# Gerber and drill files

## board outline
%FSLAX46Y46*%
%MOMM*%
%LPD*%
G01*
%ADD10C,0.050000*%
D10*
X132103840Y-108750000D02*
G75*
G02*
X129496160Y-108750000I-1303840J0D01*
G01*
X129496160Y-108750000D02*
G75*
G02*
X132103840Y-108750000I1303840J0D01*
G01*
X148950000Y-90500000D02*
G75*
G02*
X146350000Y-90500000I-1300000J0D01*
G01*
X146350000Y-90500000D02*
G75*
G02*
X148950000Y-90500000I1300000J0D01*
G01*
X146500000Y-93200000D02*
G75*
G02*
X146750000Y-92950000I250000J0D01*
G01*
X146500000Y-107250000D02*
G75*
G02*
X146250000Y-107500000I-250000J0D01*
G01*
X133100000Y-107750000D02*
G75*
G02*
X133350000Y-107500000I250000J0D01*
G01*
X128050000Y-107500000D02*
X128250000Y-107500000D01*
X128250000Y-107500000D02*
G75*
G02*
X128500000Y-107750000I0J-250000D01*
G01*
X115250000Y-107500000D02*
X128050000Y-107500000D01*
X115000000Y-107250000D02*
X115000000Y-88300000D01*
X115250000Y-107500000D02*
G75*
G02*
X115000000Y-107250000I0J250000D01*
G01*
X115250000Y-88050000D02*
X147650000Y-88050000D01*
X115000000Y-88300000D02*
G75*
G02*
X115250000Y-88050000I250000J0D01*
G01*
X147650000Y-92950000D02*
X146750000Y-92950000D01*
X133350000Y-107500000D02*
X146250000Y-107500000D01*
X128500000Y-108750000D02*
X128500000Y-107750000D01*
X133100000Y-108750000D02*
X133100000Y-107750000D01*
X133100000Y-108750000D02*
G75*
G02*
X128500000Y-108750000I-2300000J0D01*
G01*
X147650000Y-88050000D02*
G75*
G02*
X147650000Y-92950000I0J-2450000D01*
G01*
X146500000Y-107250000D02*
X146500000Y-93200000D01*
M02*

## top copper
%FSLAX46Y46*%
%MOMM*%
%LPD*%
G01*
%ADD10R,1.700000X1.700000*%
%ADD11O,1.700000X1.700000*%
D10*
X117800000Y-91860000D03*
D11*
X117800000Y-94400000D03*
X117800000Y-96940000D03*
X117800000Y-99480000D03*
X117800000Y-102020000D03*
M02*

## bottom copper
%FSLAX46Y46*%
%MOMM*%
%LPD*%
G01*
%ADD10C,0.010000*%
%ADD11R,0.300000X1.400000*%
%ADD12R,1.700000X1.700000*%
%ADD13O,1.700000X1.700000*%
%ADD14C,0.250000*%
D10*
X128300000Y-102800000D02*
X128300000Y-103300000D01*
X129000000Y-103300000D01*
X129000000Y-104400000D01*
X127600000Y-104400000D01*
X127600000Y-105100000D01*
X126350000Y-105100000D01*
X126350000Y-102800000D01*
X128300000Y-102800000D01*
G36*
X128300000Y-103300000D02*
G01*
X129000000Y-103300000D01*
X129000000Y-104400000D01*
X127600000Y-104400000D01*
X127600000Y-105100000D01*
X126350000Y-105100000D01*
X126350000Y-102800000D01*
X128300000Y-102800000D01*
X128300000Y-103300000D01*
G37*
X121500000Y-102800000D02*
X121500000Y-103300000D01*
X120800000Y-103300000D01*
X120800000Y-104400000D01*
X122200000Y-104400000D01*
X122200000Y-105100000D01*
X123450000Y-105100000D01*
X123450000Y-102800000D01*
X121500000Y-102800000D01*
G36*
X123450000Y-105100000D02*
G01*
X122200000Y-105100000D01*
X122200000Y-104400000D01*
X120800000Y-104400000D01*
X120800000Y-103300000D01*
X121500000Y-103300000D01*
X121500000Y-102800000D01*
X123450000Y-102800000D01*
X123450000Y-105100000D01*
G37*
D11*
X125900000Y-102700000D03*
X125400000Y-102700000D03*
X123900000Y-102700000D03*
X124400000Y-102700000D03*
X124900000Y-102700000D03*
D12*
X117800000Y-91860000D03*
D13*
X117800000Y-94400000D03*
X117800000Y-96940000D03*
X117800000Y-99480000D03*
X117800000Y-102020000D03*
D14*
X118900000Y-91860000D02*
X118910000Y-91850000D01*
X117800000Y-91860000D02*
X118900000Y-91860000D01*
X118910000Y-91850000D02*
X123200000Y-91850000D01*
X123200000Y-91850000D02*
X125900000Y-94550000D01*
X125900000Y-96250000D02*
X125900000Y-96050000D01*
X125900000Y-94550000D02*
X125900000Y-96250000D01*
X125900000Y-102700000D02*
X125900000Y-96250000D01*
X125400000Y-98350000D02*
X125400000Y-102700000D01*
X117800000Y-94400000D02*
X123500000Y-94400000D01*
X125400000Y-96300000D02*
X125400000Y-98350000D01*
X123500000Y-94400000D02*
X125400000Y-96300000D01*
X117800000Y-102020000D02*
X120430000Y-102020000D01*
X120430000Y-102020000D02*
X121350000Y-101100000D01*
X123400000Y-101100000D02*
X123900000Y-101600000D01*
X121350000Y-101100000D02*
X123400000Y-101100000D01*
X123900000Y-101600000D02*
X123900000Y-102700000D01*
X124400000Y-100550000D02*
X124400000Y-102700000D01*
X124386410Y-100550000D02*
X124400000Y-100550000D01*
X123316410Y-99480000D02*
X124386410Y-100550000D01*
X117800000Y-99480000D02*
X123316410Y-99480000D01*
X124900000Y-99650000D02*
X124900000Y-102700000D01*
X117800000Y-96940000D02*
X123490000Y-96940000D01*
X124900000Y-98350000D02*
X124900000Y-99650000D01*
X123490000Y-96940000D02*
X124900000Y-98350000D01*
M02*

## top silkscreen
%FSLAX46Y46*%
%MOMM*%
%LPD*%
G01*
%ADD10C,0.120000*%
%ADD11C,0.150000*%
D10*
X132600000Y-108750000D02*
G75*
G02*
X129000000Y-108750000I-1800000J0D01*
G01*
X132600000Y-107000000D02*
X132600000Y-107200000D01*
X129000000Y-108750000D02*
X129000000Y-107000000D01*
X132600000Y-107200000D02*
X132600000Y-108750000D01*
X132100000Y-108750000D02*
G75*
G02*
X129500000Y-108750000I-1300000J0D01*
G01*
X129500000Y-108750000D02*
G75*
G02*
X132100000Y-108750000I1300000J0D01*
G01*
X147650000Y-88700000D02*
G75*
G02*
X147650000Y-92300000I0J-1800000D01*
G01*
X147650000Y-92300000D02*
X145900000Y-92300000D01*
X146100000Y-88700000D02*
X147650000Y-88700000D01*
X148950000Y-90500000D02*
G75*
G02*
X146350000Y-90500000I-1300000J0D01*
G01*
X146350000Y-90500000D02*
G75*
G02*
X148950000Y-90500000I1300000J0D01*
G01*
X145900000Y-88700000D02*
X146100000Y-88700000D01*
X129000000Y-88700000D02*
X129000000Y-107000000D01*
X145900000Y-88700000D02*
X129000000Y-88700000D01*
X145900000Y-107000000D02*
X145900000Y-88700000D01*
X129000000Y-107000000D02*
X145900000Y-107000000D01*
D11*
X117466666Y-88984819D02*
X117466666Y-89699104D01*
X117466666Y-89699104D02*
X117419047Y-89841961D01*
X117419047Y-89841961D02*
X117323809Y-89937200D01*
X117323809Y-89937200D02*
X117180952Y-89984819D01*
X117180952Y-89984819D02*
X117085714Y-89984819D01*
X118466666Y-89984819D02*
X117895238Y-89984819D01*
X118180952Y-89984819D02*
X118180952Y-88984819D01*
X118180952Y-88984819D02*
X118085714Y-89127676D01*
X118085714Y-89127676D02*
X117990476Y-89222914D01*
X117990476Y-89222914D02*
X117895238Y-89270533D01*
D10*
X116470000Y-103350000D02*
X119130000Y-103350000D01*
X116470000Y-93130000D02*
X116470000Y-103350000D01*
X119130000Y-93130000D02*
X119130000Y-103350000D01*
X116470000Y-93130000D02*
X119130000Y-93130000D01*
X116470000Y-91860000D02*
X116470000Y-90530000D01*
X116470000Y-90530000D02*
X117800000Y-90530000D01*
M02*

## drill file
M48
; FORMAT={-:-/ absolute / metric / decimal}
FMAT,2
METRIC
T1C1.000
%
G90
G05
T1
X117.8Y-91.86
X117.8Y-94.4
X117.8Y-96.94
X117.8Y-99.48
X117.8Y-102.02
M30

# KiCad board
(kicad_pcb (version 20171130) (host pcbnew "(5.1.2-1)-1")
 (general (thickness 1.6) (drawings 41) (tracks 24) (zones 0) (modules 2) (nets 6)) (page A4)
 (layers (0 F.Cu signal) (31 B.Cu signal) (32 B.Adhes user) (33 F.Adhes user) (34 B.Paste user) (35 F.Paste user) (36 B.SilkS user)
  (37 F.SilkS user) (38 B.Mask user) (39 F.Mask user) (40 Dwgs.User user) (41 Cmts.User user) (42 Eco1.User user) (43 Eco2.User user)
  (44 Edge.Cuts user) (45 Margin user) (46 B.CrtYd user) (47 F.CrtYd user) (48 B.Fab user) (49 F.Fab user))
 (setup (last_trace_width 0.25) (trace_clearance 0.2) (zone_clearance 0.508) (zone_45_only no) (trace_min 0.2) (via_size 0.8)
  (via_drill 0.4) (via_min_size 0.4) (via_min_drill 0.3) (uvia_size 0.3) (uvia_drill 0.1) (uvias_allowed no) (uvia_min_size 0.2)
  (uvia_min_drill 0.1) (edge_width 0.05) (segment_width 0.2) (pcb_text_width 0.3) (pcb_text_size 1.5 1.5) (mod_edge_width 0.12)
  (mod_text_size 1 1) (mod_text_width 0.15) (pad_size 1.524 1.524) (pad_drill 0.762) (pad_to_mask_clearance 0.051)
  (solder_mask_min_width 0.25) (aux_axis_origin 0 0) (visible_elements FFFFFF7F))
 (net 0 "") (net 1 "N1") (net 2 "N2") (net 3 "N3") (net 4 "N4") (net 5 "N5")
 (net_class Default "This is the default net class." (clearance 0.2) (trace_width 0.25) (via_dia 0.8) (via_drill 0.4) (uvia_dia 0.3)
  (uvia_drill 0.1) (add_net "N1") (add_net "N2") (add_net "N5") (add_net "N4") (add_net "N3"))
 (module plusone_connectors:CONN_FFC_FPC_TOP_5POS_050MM (layer B.Cu) (at 124.9 105.2 180)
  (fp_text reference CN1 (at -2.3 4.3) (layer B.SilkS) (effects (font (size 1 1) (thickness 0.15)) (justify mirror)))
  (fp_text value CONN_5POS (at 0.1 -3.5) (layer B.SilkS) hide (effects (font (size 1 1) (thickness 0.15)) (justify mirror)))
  (fp_poly
   (pts (xy -3.4 2.4) (xy -3.4 1.9) (xy -4.1 1.9) (xy -4.1 0.8) (xy -2.7 0.8) (xy -2.7 0.1) (xy -1.45 0.1) (xy -1.45 2.4)) (layer B.Cu)
   (width 0.01))
  (fp_poly
   (pts (xy 3.4 2.4) (xy 3.4 1.9) (xy 4.1 1.9) (xy 4.1 0.8) (xy 2.7 0.8) (xy 2.7 0.1) (xy 1.45 0.1) (xy 1.45 2.4)) (layer B.Cu) (width 0.01))
  (pad 1 smd rect (at -1 2.5 180) (size 0.3 1.4) (layers B.Cu B.Paste B.Mask) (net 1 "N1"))
  (pad 2 smd rect (at -0.5 2.5 180) (size 0.3 1.4) (layers B.Cu B.Paste B.Mask) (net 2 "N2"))
  (pad 5 smd rect (at 1 2.5 180) (size 0.3 1.4) (layers B.Cu B.Paste B.Mask) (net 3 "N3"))
  (pad 4 smd rect (at 0.5 2.5 180) (size 0.3 1.4) (layers B.Cu B.Paste B.Mask) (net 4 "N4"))
  (pad 3 smd rect (at 0 2.5 180) (size 0.3 1.4) (layers B.Cu B.Paste B.Mask) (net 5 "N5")))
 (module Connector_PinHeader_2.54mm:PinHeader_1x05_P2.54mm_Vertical (layer F.Cu) (at 117.8 91.86)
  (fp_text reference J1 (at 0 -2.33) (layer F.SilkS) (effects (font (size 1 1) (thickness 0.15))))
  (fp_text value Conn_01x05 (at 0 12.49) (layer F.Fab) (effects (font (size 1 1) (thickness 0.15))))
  (fp_line (start -1.33 11.49) (end 1.33 11.49) (layer F.SilkS) (width 0.12))
  (fp_line (start -1.33 1.27) (end -1.33 11.49) (layer F.SilkS) (width 0.12))
  (fp_line (start 1.33 1.27) (end 1.33 11.49) (layer F.SilkS) (width 0.12))
  (fp_line (start -1.33 1.27) (end 1.33 1.27) (layer F.SilkS) (width 0.12))
  (fp_line (start -1.33 0) (end -1.33 -1.33) (layer F.SilkS) (width 0.12))
  (fp_line (start -1.33 -1.33) (end 0 -1.33) (layer F.SilkS) (width 0.12))
  (pad 1 thru_hole rect (at 0 0) (size 1.7 1.7) (drill 1) (layers *.Cu *.Mask) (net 1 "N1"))
  (pad 2 thru_hole oval (at 0 2.54) (size 1.7 1.7) (drill 1) (layers *.Cu *.Mask) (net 2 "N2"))
  (pad 3 thru_hole oval (at 0 5.08) (size 1.7 1.7) (drill 1) (layers *.Cu *.Mask) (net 5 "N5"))
  (pad 4 thru_hole oval (at 0 7.62) (size 1.7 1.7) (drill 1) (layers *.Cu *.Mask) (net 4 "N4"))
  (pad 5 thru_hole oval (at 0 10.16) (size 1.7 1.7) (drill 1) (layers *.Cu *.Mask) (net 3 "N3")))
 (gr_circle (center 130.8 108.75) (end 129.7 109.45) (layer Edge.Cuts) (width 0.05))
 (gr_circle (center 147.65 90.5) (end 148.95 90.5) (layer Edge.Cuts) (width 0.05))
 (gr_arc (start 146.75 93.2) (end 146.75 92.95) (angle -90) (layer Edge.Cuts) (width 0.05))
 (gr_arc (start 146.25 107.25) (end 146.25 107.5) (angle -90) (layer Edge.Cuts) (width 0.05))
 (gr_arc (start 133.35 107.75) (end 133.35 107.5) (angle -90) (layer Edge.Cuts) (width 0.05))
 (gr_line (start 128.05 107.5) (end 128.25 107.5) (layer Edge.Cuts) (width 0.05))
 (gr_arc (start 128.25 107.75) (end 128.5 107.75) (angle -90) (layer Edge.Cuts) (width 0.05))
 (gr_line (start 115.25 107.5) (end 128.05 107.5) (layer Edge.Cuts) (width 0.05))
 (gr_line (start 115 107.25) (end 115 88.3) (layer Edge.Cuts) (width 0.05))
 (gr_arc (start 115.25 107.25) (end 115 107.25) (angle -90) (layer Edge.Cuts) (width 0.05))
 (gr_line (start 115.25 88.05) (end 147.65 88.05) (layer Edge.Cuts) (width 0.05))
 (gr_arc (start 115.25 88.3) (end 115.25 88.05) (angle -90) (layer Edge.Cuts) (width 0.05))
 (gr_line (start 147.65 92.95) (end 146.75 92.95) (layer Edge.Cuts) (width 0.05))
 (gr_line (start 133.35 107.5) (end 146.25 107.5) (layer Edge.Cuts) (width 0.05))
 (gr_line (start 128.5 108.75) (end 128.5 107.75) (layer Edge.Cuts) (width 0.05))
 (gr_line (start 133.1 108.75) (end 133.1 107.75) (layer Edge.Cuts) (width 0.05))
 (gr_arc (start 130.8 108.75) (end 128.5 108.75) (angle -180) (layer Edge.Cuts) (width 0.05))
 (gr_arc (start 147.65 90.5) (end 147.65 92.95) (angle -180) (layer Edge.Cuts) (width 0.05))
 (gr_line (start 146.5 107.25) (end 146.5 93.2) (layer Edge.Cuts) (width 0.05))
 (gr_arc (start 130.8 108.75) (end 129 108.75) (angle -180) (layer F.SilkS) (width 0.12))
 (gr_line (start 132.6 107) (end 132.6 107.2) (layer F.SilkS) (width 0.12))
 (gr_line (start 129 108.75) (end 129 107) (layer F.SilkS) (width 0.12))
 (gr_line (start 132.6 107.2) (end 132.6 108.75) (layer F.SilkS) (width 0.12))
 (gr_circle (center 130.8 108.75) (end 130.8 110.05) (layer F.SilkS) (width 0.12))
 (gr_arc (start 147.65 90.5) (end 147.65 92.3) (angle -180) (layer F.SilkS) (width 0.12))
 (gr_line (start 147.65 92.3) (end 145.9 92.3) (layer F.SilkS) (width 0.12))
 (gr_line (start 146.1 88.7) (end 147.65 88.7) (layer F.SilkS) (width 0.12))
 (gr_circle (center 147.65 90.5) (end 148.95 90.5) (layer F.SilkS) (width 0.12))
 (gr_line (start 145.9 88.7) (end 146.1 88.7) (layer F.SilkS) (width 0.12))
 (gr_line (start 129 88.7) (end 129 107) (layer F.SilkS) (width 0.12))
 (gr_line (start 145.9 88.7) (end 129 88.7) (layer F.SilkS) (width 0.12))
 (gr_line (start 145.9 107) (end 145.9 88.7) (layer F.SilkS) (width 0.12))
 (gr_line (start 129 107) (end 145.9 107) (layer F.SilkS) (width 0.12))
 (segment (start 118.9 91.86) (end 118.91 91.85) (width 0.25) (layer B.Cu) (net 1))
 (segment (start 117.8 91.86) (end 118.9 91.86) (width 0.25) (layer B.Cu) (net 1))
 (segment (start 118.91 91.85) (end 123.2 91.85) (width 0.25) (layer B.Cu) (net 1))
 (segment (start 123.2 91.85) (end 125.9 94.55) (width 0.25) (layer B.Cu) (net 1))
 (segment (start 125.9 96.25) (end 125.9 96.05) (width 0.25) (layer B.Cu) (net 1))
 (segment (start 125.9 94.55) (end 125.9 96.25) (width 0.25) (layer B.Cu) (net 1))
 (segment (start 125.9 102.7) (end 125.9 96.25) (width 0.25) (layer B.Cu) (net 1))
 (segment (start 125.4 98.35) (end 125.4 102.7) (width 0.25) (layer B.Cu) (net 2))
 (segment (start 117.8 94.4) (end 123.5 94.4) (width 0.25) (layer B.Cu) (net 2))
 (segment (start 125.4 96.3) (end 125.4 98.35) (width 0.25) (layer B.Cu) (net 2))
 (segment (start 123.5 94.4) (end 125.4 96.3) (width 0.25) (layer B.Cu) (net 2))
 (segment (start 117.8 102.02) (end 120.43 102.02) (width 0.25) (layer B.Cu) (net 3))
 (segment (start 120.43 102.02) (end 121.35 101.1) (width 0.25) (layer B.Cu) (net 3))
 (segment (start 123.4 101.1) (end 123.9 101.6) (width 0.25) (layer B.Cu) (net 3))
 (segment (start 121.35 101.1) (end 123.4 101.1) (width 0.25) (layer B.Cu) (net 3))
 (segment (start 123.9 101.6) (end 123.9 102.7) (width 0.25) (layer B.Cu) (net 3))
 (segment (start 124.4 100.55) (end 124.4 102.7) (width 0.25) (layer B.Cu) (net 4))
 (segment (start 124.38641 100.55) (end 124.4 100.55) (width 0.25) (layer B.Cu) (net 4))
 (segment (start 123.31641 99.48) (end 124.38641 100.55) (width 0.25) (layer B.Cu) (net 4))
 (segment (start 117.8 99.48) (end 123.31641 99.48) (width 0.25) (layer B.Cu) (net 4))
 (segment (start 124.9 99.65) (end 124.9 102.7) (width 0.25) (layer B.Cu) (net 5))
 (segment (start 117.8 96.94) (end 123.49 96.94) (width 0.25) (layer B.Cu) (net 5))
 (segment (start 124.9 98.35) (end 124.9 99.65) (width 0.25) (layer B.Cu) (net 5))
 (segment (start 123.49 96.94) (end 124.9 98.35) (width 0.25) (layer B.Cu) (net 5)))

